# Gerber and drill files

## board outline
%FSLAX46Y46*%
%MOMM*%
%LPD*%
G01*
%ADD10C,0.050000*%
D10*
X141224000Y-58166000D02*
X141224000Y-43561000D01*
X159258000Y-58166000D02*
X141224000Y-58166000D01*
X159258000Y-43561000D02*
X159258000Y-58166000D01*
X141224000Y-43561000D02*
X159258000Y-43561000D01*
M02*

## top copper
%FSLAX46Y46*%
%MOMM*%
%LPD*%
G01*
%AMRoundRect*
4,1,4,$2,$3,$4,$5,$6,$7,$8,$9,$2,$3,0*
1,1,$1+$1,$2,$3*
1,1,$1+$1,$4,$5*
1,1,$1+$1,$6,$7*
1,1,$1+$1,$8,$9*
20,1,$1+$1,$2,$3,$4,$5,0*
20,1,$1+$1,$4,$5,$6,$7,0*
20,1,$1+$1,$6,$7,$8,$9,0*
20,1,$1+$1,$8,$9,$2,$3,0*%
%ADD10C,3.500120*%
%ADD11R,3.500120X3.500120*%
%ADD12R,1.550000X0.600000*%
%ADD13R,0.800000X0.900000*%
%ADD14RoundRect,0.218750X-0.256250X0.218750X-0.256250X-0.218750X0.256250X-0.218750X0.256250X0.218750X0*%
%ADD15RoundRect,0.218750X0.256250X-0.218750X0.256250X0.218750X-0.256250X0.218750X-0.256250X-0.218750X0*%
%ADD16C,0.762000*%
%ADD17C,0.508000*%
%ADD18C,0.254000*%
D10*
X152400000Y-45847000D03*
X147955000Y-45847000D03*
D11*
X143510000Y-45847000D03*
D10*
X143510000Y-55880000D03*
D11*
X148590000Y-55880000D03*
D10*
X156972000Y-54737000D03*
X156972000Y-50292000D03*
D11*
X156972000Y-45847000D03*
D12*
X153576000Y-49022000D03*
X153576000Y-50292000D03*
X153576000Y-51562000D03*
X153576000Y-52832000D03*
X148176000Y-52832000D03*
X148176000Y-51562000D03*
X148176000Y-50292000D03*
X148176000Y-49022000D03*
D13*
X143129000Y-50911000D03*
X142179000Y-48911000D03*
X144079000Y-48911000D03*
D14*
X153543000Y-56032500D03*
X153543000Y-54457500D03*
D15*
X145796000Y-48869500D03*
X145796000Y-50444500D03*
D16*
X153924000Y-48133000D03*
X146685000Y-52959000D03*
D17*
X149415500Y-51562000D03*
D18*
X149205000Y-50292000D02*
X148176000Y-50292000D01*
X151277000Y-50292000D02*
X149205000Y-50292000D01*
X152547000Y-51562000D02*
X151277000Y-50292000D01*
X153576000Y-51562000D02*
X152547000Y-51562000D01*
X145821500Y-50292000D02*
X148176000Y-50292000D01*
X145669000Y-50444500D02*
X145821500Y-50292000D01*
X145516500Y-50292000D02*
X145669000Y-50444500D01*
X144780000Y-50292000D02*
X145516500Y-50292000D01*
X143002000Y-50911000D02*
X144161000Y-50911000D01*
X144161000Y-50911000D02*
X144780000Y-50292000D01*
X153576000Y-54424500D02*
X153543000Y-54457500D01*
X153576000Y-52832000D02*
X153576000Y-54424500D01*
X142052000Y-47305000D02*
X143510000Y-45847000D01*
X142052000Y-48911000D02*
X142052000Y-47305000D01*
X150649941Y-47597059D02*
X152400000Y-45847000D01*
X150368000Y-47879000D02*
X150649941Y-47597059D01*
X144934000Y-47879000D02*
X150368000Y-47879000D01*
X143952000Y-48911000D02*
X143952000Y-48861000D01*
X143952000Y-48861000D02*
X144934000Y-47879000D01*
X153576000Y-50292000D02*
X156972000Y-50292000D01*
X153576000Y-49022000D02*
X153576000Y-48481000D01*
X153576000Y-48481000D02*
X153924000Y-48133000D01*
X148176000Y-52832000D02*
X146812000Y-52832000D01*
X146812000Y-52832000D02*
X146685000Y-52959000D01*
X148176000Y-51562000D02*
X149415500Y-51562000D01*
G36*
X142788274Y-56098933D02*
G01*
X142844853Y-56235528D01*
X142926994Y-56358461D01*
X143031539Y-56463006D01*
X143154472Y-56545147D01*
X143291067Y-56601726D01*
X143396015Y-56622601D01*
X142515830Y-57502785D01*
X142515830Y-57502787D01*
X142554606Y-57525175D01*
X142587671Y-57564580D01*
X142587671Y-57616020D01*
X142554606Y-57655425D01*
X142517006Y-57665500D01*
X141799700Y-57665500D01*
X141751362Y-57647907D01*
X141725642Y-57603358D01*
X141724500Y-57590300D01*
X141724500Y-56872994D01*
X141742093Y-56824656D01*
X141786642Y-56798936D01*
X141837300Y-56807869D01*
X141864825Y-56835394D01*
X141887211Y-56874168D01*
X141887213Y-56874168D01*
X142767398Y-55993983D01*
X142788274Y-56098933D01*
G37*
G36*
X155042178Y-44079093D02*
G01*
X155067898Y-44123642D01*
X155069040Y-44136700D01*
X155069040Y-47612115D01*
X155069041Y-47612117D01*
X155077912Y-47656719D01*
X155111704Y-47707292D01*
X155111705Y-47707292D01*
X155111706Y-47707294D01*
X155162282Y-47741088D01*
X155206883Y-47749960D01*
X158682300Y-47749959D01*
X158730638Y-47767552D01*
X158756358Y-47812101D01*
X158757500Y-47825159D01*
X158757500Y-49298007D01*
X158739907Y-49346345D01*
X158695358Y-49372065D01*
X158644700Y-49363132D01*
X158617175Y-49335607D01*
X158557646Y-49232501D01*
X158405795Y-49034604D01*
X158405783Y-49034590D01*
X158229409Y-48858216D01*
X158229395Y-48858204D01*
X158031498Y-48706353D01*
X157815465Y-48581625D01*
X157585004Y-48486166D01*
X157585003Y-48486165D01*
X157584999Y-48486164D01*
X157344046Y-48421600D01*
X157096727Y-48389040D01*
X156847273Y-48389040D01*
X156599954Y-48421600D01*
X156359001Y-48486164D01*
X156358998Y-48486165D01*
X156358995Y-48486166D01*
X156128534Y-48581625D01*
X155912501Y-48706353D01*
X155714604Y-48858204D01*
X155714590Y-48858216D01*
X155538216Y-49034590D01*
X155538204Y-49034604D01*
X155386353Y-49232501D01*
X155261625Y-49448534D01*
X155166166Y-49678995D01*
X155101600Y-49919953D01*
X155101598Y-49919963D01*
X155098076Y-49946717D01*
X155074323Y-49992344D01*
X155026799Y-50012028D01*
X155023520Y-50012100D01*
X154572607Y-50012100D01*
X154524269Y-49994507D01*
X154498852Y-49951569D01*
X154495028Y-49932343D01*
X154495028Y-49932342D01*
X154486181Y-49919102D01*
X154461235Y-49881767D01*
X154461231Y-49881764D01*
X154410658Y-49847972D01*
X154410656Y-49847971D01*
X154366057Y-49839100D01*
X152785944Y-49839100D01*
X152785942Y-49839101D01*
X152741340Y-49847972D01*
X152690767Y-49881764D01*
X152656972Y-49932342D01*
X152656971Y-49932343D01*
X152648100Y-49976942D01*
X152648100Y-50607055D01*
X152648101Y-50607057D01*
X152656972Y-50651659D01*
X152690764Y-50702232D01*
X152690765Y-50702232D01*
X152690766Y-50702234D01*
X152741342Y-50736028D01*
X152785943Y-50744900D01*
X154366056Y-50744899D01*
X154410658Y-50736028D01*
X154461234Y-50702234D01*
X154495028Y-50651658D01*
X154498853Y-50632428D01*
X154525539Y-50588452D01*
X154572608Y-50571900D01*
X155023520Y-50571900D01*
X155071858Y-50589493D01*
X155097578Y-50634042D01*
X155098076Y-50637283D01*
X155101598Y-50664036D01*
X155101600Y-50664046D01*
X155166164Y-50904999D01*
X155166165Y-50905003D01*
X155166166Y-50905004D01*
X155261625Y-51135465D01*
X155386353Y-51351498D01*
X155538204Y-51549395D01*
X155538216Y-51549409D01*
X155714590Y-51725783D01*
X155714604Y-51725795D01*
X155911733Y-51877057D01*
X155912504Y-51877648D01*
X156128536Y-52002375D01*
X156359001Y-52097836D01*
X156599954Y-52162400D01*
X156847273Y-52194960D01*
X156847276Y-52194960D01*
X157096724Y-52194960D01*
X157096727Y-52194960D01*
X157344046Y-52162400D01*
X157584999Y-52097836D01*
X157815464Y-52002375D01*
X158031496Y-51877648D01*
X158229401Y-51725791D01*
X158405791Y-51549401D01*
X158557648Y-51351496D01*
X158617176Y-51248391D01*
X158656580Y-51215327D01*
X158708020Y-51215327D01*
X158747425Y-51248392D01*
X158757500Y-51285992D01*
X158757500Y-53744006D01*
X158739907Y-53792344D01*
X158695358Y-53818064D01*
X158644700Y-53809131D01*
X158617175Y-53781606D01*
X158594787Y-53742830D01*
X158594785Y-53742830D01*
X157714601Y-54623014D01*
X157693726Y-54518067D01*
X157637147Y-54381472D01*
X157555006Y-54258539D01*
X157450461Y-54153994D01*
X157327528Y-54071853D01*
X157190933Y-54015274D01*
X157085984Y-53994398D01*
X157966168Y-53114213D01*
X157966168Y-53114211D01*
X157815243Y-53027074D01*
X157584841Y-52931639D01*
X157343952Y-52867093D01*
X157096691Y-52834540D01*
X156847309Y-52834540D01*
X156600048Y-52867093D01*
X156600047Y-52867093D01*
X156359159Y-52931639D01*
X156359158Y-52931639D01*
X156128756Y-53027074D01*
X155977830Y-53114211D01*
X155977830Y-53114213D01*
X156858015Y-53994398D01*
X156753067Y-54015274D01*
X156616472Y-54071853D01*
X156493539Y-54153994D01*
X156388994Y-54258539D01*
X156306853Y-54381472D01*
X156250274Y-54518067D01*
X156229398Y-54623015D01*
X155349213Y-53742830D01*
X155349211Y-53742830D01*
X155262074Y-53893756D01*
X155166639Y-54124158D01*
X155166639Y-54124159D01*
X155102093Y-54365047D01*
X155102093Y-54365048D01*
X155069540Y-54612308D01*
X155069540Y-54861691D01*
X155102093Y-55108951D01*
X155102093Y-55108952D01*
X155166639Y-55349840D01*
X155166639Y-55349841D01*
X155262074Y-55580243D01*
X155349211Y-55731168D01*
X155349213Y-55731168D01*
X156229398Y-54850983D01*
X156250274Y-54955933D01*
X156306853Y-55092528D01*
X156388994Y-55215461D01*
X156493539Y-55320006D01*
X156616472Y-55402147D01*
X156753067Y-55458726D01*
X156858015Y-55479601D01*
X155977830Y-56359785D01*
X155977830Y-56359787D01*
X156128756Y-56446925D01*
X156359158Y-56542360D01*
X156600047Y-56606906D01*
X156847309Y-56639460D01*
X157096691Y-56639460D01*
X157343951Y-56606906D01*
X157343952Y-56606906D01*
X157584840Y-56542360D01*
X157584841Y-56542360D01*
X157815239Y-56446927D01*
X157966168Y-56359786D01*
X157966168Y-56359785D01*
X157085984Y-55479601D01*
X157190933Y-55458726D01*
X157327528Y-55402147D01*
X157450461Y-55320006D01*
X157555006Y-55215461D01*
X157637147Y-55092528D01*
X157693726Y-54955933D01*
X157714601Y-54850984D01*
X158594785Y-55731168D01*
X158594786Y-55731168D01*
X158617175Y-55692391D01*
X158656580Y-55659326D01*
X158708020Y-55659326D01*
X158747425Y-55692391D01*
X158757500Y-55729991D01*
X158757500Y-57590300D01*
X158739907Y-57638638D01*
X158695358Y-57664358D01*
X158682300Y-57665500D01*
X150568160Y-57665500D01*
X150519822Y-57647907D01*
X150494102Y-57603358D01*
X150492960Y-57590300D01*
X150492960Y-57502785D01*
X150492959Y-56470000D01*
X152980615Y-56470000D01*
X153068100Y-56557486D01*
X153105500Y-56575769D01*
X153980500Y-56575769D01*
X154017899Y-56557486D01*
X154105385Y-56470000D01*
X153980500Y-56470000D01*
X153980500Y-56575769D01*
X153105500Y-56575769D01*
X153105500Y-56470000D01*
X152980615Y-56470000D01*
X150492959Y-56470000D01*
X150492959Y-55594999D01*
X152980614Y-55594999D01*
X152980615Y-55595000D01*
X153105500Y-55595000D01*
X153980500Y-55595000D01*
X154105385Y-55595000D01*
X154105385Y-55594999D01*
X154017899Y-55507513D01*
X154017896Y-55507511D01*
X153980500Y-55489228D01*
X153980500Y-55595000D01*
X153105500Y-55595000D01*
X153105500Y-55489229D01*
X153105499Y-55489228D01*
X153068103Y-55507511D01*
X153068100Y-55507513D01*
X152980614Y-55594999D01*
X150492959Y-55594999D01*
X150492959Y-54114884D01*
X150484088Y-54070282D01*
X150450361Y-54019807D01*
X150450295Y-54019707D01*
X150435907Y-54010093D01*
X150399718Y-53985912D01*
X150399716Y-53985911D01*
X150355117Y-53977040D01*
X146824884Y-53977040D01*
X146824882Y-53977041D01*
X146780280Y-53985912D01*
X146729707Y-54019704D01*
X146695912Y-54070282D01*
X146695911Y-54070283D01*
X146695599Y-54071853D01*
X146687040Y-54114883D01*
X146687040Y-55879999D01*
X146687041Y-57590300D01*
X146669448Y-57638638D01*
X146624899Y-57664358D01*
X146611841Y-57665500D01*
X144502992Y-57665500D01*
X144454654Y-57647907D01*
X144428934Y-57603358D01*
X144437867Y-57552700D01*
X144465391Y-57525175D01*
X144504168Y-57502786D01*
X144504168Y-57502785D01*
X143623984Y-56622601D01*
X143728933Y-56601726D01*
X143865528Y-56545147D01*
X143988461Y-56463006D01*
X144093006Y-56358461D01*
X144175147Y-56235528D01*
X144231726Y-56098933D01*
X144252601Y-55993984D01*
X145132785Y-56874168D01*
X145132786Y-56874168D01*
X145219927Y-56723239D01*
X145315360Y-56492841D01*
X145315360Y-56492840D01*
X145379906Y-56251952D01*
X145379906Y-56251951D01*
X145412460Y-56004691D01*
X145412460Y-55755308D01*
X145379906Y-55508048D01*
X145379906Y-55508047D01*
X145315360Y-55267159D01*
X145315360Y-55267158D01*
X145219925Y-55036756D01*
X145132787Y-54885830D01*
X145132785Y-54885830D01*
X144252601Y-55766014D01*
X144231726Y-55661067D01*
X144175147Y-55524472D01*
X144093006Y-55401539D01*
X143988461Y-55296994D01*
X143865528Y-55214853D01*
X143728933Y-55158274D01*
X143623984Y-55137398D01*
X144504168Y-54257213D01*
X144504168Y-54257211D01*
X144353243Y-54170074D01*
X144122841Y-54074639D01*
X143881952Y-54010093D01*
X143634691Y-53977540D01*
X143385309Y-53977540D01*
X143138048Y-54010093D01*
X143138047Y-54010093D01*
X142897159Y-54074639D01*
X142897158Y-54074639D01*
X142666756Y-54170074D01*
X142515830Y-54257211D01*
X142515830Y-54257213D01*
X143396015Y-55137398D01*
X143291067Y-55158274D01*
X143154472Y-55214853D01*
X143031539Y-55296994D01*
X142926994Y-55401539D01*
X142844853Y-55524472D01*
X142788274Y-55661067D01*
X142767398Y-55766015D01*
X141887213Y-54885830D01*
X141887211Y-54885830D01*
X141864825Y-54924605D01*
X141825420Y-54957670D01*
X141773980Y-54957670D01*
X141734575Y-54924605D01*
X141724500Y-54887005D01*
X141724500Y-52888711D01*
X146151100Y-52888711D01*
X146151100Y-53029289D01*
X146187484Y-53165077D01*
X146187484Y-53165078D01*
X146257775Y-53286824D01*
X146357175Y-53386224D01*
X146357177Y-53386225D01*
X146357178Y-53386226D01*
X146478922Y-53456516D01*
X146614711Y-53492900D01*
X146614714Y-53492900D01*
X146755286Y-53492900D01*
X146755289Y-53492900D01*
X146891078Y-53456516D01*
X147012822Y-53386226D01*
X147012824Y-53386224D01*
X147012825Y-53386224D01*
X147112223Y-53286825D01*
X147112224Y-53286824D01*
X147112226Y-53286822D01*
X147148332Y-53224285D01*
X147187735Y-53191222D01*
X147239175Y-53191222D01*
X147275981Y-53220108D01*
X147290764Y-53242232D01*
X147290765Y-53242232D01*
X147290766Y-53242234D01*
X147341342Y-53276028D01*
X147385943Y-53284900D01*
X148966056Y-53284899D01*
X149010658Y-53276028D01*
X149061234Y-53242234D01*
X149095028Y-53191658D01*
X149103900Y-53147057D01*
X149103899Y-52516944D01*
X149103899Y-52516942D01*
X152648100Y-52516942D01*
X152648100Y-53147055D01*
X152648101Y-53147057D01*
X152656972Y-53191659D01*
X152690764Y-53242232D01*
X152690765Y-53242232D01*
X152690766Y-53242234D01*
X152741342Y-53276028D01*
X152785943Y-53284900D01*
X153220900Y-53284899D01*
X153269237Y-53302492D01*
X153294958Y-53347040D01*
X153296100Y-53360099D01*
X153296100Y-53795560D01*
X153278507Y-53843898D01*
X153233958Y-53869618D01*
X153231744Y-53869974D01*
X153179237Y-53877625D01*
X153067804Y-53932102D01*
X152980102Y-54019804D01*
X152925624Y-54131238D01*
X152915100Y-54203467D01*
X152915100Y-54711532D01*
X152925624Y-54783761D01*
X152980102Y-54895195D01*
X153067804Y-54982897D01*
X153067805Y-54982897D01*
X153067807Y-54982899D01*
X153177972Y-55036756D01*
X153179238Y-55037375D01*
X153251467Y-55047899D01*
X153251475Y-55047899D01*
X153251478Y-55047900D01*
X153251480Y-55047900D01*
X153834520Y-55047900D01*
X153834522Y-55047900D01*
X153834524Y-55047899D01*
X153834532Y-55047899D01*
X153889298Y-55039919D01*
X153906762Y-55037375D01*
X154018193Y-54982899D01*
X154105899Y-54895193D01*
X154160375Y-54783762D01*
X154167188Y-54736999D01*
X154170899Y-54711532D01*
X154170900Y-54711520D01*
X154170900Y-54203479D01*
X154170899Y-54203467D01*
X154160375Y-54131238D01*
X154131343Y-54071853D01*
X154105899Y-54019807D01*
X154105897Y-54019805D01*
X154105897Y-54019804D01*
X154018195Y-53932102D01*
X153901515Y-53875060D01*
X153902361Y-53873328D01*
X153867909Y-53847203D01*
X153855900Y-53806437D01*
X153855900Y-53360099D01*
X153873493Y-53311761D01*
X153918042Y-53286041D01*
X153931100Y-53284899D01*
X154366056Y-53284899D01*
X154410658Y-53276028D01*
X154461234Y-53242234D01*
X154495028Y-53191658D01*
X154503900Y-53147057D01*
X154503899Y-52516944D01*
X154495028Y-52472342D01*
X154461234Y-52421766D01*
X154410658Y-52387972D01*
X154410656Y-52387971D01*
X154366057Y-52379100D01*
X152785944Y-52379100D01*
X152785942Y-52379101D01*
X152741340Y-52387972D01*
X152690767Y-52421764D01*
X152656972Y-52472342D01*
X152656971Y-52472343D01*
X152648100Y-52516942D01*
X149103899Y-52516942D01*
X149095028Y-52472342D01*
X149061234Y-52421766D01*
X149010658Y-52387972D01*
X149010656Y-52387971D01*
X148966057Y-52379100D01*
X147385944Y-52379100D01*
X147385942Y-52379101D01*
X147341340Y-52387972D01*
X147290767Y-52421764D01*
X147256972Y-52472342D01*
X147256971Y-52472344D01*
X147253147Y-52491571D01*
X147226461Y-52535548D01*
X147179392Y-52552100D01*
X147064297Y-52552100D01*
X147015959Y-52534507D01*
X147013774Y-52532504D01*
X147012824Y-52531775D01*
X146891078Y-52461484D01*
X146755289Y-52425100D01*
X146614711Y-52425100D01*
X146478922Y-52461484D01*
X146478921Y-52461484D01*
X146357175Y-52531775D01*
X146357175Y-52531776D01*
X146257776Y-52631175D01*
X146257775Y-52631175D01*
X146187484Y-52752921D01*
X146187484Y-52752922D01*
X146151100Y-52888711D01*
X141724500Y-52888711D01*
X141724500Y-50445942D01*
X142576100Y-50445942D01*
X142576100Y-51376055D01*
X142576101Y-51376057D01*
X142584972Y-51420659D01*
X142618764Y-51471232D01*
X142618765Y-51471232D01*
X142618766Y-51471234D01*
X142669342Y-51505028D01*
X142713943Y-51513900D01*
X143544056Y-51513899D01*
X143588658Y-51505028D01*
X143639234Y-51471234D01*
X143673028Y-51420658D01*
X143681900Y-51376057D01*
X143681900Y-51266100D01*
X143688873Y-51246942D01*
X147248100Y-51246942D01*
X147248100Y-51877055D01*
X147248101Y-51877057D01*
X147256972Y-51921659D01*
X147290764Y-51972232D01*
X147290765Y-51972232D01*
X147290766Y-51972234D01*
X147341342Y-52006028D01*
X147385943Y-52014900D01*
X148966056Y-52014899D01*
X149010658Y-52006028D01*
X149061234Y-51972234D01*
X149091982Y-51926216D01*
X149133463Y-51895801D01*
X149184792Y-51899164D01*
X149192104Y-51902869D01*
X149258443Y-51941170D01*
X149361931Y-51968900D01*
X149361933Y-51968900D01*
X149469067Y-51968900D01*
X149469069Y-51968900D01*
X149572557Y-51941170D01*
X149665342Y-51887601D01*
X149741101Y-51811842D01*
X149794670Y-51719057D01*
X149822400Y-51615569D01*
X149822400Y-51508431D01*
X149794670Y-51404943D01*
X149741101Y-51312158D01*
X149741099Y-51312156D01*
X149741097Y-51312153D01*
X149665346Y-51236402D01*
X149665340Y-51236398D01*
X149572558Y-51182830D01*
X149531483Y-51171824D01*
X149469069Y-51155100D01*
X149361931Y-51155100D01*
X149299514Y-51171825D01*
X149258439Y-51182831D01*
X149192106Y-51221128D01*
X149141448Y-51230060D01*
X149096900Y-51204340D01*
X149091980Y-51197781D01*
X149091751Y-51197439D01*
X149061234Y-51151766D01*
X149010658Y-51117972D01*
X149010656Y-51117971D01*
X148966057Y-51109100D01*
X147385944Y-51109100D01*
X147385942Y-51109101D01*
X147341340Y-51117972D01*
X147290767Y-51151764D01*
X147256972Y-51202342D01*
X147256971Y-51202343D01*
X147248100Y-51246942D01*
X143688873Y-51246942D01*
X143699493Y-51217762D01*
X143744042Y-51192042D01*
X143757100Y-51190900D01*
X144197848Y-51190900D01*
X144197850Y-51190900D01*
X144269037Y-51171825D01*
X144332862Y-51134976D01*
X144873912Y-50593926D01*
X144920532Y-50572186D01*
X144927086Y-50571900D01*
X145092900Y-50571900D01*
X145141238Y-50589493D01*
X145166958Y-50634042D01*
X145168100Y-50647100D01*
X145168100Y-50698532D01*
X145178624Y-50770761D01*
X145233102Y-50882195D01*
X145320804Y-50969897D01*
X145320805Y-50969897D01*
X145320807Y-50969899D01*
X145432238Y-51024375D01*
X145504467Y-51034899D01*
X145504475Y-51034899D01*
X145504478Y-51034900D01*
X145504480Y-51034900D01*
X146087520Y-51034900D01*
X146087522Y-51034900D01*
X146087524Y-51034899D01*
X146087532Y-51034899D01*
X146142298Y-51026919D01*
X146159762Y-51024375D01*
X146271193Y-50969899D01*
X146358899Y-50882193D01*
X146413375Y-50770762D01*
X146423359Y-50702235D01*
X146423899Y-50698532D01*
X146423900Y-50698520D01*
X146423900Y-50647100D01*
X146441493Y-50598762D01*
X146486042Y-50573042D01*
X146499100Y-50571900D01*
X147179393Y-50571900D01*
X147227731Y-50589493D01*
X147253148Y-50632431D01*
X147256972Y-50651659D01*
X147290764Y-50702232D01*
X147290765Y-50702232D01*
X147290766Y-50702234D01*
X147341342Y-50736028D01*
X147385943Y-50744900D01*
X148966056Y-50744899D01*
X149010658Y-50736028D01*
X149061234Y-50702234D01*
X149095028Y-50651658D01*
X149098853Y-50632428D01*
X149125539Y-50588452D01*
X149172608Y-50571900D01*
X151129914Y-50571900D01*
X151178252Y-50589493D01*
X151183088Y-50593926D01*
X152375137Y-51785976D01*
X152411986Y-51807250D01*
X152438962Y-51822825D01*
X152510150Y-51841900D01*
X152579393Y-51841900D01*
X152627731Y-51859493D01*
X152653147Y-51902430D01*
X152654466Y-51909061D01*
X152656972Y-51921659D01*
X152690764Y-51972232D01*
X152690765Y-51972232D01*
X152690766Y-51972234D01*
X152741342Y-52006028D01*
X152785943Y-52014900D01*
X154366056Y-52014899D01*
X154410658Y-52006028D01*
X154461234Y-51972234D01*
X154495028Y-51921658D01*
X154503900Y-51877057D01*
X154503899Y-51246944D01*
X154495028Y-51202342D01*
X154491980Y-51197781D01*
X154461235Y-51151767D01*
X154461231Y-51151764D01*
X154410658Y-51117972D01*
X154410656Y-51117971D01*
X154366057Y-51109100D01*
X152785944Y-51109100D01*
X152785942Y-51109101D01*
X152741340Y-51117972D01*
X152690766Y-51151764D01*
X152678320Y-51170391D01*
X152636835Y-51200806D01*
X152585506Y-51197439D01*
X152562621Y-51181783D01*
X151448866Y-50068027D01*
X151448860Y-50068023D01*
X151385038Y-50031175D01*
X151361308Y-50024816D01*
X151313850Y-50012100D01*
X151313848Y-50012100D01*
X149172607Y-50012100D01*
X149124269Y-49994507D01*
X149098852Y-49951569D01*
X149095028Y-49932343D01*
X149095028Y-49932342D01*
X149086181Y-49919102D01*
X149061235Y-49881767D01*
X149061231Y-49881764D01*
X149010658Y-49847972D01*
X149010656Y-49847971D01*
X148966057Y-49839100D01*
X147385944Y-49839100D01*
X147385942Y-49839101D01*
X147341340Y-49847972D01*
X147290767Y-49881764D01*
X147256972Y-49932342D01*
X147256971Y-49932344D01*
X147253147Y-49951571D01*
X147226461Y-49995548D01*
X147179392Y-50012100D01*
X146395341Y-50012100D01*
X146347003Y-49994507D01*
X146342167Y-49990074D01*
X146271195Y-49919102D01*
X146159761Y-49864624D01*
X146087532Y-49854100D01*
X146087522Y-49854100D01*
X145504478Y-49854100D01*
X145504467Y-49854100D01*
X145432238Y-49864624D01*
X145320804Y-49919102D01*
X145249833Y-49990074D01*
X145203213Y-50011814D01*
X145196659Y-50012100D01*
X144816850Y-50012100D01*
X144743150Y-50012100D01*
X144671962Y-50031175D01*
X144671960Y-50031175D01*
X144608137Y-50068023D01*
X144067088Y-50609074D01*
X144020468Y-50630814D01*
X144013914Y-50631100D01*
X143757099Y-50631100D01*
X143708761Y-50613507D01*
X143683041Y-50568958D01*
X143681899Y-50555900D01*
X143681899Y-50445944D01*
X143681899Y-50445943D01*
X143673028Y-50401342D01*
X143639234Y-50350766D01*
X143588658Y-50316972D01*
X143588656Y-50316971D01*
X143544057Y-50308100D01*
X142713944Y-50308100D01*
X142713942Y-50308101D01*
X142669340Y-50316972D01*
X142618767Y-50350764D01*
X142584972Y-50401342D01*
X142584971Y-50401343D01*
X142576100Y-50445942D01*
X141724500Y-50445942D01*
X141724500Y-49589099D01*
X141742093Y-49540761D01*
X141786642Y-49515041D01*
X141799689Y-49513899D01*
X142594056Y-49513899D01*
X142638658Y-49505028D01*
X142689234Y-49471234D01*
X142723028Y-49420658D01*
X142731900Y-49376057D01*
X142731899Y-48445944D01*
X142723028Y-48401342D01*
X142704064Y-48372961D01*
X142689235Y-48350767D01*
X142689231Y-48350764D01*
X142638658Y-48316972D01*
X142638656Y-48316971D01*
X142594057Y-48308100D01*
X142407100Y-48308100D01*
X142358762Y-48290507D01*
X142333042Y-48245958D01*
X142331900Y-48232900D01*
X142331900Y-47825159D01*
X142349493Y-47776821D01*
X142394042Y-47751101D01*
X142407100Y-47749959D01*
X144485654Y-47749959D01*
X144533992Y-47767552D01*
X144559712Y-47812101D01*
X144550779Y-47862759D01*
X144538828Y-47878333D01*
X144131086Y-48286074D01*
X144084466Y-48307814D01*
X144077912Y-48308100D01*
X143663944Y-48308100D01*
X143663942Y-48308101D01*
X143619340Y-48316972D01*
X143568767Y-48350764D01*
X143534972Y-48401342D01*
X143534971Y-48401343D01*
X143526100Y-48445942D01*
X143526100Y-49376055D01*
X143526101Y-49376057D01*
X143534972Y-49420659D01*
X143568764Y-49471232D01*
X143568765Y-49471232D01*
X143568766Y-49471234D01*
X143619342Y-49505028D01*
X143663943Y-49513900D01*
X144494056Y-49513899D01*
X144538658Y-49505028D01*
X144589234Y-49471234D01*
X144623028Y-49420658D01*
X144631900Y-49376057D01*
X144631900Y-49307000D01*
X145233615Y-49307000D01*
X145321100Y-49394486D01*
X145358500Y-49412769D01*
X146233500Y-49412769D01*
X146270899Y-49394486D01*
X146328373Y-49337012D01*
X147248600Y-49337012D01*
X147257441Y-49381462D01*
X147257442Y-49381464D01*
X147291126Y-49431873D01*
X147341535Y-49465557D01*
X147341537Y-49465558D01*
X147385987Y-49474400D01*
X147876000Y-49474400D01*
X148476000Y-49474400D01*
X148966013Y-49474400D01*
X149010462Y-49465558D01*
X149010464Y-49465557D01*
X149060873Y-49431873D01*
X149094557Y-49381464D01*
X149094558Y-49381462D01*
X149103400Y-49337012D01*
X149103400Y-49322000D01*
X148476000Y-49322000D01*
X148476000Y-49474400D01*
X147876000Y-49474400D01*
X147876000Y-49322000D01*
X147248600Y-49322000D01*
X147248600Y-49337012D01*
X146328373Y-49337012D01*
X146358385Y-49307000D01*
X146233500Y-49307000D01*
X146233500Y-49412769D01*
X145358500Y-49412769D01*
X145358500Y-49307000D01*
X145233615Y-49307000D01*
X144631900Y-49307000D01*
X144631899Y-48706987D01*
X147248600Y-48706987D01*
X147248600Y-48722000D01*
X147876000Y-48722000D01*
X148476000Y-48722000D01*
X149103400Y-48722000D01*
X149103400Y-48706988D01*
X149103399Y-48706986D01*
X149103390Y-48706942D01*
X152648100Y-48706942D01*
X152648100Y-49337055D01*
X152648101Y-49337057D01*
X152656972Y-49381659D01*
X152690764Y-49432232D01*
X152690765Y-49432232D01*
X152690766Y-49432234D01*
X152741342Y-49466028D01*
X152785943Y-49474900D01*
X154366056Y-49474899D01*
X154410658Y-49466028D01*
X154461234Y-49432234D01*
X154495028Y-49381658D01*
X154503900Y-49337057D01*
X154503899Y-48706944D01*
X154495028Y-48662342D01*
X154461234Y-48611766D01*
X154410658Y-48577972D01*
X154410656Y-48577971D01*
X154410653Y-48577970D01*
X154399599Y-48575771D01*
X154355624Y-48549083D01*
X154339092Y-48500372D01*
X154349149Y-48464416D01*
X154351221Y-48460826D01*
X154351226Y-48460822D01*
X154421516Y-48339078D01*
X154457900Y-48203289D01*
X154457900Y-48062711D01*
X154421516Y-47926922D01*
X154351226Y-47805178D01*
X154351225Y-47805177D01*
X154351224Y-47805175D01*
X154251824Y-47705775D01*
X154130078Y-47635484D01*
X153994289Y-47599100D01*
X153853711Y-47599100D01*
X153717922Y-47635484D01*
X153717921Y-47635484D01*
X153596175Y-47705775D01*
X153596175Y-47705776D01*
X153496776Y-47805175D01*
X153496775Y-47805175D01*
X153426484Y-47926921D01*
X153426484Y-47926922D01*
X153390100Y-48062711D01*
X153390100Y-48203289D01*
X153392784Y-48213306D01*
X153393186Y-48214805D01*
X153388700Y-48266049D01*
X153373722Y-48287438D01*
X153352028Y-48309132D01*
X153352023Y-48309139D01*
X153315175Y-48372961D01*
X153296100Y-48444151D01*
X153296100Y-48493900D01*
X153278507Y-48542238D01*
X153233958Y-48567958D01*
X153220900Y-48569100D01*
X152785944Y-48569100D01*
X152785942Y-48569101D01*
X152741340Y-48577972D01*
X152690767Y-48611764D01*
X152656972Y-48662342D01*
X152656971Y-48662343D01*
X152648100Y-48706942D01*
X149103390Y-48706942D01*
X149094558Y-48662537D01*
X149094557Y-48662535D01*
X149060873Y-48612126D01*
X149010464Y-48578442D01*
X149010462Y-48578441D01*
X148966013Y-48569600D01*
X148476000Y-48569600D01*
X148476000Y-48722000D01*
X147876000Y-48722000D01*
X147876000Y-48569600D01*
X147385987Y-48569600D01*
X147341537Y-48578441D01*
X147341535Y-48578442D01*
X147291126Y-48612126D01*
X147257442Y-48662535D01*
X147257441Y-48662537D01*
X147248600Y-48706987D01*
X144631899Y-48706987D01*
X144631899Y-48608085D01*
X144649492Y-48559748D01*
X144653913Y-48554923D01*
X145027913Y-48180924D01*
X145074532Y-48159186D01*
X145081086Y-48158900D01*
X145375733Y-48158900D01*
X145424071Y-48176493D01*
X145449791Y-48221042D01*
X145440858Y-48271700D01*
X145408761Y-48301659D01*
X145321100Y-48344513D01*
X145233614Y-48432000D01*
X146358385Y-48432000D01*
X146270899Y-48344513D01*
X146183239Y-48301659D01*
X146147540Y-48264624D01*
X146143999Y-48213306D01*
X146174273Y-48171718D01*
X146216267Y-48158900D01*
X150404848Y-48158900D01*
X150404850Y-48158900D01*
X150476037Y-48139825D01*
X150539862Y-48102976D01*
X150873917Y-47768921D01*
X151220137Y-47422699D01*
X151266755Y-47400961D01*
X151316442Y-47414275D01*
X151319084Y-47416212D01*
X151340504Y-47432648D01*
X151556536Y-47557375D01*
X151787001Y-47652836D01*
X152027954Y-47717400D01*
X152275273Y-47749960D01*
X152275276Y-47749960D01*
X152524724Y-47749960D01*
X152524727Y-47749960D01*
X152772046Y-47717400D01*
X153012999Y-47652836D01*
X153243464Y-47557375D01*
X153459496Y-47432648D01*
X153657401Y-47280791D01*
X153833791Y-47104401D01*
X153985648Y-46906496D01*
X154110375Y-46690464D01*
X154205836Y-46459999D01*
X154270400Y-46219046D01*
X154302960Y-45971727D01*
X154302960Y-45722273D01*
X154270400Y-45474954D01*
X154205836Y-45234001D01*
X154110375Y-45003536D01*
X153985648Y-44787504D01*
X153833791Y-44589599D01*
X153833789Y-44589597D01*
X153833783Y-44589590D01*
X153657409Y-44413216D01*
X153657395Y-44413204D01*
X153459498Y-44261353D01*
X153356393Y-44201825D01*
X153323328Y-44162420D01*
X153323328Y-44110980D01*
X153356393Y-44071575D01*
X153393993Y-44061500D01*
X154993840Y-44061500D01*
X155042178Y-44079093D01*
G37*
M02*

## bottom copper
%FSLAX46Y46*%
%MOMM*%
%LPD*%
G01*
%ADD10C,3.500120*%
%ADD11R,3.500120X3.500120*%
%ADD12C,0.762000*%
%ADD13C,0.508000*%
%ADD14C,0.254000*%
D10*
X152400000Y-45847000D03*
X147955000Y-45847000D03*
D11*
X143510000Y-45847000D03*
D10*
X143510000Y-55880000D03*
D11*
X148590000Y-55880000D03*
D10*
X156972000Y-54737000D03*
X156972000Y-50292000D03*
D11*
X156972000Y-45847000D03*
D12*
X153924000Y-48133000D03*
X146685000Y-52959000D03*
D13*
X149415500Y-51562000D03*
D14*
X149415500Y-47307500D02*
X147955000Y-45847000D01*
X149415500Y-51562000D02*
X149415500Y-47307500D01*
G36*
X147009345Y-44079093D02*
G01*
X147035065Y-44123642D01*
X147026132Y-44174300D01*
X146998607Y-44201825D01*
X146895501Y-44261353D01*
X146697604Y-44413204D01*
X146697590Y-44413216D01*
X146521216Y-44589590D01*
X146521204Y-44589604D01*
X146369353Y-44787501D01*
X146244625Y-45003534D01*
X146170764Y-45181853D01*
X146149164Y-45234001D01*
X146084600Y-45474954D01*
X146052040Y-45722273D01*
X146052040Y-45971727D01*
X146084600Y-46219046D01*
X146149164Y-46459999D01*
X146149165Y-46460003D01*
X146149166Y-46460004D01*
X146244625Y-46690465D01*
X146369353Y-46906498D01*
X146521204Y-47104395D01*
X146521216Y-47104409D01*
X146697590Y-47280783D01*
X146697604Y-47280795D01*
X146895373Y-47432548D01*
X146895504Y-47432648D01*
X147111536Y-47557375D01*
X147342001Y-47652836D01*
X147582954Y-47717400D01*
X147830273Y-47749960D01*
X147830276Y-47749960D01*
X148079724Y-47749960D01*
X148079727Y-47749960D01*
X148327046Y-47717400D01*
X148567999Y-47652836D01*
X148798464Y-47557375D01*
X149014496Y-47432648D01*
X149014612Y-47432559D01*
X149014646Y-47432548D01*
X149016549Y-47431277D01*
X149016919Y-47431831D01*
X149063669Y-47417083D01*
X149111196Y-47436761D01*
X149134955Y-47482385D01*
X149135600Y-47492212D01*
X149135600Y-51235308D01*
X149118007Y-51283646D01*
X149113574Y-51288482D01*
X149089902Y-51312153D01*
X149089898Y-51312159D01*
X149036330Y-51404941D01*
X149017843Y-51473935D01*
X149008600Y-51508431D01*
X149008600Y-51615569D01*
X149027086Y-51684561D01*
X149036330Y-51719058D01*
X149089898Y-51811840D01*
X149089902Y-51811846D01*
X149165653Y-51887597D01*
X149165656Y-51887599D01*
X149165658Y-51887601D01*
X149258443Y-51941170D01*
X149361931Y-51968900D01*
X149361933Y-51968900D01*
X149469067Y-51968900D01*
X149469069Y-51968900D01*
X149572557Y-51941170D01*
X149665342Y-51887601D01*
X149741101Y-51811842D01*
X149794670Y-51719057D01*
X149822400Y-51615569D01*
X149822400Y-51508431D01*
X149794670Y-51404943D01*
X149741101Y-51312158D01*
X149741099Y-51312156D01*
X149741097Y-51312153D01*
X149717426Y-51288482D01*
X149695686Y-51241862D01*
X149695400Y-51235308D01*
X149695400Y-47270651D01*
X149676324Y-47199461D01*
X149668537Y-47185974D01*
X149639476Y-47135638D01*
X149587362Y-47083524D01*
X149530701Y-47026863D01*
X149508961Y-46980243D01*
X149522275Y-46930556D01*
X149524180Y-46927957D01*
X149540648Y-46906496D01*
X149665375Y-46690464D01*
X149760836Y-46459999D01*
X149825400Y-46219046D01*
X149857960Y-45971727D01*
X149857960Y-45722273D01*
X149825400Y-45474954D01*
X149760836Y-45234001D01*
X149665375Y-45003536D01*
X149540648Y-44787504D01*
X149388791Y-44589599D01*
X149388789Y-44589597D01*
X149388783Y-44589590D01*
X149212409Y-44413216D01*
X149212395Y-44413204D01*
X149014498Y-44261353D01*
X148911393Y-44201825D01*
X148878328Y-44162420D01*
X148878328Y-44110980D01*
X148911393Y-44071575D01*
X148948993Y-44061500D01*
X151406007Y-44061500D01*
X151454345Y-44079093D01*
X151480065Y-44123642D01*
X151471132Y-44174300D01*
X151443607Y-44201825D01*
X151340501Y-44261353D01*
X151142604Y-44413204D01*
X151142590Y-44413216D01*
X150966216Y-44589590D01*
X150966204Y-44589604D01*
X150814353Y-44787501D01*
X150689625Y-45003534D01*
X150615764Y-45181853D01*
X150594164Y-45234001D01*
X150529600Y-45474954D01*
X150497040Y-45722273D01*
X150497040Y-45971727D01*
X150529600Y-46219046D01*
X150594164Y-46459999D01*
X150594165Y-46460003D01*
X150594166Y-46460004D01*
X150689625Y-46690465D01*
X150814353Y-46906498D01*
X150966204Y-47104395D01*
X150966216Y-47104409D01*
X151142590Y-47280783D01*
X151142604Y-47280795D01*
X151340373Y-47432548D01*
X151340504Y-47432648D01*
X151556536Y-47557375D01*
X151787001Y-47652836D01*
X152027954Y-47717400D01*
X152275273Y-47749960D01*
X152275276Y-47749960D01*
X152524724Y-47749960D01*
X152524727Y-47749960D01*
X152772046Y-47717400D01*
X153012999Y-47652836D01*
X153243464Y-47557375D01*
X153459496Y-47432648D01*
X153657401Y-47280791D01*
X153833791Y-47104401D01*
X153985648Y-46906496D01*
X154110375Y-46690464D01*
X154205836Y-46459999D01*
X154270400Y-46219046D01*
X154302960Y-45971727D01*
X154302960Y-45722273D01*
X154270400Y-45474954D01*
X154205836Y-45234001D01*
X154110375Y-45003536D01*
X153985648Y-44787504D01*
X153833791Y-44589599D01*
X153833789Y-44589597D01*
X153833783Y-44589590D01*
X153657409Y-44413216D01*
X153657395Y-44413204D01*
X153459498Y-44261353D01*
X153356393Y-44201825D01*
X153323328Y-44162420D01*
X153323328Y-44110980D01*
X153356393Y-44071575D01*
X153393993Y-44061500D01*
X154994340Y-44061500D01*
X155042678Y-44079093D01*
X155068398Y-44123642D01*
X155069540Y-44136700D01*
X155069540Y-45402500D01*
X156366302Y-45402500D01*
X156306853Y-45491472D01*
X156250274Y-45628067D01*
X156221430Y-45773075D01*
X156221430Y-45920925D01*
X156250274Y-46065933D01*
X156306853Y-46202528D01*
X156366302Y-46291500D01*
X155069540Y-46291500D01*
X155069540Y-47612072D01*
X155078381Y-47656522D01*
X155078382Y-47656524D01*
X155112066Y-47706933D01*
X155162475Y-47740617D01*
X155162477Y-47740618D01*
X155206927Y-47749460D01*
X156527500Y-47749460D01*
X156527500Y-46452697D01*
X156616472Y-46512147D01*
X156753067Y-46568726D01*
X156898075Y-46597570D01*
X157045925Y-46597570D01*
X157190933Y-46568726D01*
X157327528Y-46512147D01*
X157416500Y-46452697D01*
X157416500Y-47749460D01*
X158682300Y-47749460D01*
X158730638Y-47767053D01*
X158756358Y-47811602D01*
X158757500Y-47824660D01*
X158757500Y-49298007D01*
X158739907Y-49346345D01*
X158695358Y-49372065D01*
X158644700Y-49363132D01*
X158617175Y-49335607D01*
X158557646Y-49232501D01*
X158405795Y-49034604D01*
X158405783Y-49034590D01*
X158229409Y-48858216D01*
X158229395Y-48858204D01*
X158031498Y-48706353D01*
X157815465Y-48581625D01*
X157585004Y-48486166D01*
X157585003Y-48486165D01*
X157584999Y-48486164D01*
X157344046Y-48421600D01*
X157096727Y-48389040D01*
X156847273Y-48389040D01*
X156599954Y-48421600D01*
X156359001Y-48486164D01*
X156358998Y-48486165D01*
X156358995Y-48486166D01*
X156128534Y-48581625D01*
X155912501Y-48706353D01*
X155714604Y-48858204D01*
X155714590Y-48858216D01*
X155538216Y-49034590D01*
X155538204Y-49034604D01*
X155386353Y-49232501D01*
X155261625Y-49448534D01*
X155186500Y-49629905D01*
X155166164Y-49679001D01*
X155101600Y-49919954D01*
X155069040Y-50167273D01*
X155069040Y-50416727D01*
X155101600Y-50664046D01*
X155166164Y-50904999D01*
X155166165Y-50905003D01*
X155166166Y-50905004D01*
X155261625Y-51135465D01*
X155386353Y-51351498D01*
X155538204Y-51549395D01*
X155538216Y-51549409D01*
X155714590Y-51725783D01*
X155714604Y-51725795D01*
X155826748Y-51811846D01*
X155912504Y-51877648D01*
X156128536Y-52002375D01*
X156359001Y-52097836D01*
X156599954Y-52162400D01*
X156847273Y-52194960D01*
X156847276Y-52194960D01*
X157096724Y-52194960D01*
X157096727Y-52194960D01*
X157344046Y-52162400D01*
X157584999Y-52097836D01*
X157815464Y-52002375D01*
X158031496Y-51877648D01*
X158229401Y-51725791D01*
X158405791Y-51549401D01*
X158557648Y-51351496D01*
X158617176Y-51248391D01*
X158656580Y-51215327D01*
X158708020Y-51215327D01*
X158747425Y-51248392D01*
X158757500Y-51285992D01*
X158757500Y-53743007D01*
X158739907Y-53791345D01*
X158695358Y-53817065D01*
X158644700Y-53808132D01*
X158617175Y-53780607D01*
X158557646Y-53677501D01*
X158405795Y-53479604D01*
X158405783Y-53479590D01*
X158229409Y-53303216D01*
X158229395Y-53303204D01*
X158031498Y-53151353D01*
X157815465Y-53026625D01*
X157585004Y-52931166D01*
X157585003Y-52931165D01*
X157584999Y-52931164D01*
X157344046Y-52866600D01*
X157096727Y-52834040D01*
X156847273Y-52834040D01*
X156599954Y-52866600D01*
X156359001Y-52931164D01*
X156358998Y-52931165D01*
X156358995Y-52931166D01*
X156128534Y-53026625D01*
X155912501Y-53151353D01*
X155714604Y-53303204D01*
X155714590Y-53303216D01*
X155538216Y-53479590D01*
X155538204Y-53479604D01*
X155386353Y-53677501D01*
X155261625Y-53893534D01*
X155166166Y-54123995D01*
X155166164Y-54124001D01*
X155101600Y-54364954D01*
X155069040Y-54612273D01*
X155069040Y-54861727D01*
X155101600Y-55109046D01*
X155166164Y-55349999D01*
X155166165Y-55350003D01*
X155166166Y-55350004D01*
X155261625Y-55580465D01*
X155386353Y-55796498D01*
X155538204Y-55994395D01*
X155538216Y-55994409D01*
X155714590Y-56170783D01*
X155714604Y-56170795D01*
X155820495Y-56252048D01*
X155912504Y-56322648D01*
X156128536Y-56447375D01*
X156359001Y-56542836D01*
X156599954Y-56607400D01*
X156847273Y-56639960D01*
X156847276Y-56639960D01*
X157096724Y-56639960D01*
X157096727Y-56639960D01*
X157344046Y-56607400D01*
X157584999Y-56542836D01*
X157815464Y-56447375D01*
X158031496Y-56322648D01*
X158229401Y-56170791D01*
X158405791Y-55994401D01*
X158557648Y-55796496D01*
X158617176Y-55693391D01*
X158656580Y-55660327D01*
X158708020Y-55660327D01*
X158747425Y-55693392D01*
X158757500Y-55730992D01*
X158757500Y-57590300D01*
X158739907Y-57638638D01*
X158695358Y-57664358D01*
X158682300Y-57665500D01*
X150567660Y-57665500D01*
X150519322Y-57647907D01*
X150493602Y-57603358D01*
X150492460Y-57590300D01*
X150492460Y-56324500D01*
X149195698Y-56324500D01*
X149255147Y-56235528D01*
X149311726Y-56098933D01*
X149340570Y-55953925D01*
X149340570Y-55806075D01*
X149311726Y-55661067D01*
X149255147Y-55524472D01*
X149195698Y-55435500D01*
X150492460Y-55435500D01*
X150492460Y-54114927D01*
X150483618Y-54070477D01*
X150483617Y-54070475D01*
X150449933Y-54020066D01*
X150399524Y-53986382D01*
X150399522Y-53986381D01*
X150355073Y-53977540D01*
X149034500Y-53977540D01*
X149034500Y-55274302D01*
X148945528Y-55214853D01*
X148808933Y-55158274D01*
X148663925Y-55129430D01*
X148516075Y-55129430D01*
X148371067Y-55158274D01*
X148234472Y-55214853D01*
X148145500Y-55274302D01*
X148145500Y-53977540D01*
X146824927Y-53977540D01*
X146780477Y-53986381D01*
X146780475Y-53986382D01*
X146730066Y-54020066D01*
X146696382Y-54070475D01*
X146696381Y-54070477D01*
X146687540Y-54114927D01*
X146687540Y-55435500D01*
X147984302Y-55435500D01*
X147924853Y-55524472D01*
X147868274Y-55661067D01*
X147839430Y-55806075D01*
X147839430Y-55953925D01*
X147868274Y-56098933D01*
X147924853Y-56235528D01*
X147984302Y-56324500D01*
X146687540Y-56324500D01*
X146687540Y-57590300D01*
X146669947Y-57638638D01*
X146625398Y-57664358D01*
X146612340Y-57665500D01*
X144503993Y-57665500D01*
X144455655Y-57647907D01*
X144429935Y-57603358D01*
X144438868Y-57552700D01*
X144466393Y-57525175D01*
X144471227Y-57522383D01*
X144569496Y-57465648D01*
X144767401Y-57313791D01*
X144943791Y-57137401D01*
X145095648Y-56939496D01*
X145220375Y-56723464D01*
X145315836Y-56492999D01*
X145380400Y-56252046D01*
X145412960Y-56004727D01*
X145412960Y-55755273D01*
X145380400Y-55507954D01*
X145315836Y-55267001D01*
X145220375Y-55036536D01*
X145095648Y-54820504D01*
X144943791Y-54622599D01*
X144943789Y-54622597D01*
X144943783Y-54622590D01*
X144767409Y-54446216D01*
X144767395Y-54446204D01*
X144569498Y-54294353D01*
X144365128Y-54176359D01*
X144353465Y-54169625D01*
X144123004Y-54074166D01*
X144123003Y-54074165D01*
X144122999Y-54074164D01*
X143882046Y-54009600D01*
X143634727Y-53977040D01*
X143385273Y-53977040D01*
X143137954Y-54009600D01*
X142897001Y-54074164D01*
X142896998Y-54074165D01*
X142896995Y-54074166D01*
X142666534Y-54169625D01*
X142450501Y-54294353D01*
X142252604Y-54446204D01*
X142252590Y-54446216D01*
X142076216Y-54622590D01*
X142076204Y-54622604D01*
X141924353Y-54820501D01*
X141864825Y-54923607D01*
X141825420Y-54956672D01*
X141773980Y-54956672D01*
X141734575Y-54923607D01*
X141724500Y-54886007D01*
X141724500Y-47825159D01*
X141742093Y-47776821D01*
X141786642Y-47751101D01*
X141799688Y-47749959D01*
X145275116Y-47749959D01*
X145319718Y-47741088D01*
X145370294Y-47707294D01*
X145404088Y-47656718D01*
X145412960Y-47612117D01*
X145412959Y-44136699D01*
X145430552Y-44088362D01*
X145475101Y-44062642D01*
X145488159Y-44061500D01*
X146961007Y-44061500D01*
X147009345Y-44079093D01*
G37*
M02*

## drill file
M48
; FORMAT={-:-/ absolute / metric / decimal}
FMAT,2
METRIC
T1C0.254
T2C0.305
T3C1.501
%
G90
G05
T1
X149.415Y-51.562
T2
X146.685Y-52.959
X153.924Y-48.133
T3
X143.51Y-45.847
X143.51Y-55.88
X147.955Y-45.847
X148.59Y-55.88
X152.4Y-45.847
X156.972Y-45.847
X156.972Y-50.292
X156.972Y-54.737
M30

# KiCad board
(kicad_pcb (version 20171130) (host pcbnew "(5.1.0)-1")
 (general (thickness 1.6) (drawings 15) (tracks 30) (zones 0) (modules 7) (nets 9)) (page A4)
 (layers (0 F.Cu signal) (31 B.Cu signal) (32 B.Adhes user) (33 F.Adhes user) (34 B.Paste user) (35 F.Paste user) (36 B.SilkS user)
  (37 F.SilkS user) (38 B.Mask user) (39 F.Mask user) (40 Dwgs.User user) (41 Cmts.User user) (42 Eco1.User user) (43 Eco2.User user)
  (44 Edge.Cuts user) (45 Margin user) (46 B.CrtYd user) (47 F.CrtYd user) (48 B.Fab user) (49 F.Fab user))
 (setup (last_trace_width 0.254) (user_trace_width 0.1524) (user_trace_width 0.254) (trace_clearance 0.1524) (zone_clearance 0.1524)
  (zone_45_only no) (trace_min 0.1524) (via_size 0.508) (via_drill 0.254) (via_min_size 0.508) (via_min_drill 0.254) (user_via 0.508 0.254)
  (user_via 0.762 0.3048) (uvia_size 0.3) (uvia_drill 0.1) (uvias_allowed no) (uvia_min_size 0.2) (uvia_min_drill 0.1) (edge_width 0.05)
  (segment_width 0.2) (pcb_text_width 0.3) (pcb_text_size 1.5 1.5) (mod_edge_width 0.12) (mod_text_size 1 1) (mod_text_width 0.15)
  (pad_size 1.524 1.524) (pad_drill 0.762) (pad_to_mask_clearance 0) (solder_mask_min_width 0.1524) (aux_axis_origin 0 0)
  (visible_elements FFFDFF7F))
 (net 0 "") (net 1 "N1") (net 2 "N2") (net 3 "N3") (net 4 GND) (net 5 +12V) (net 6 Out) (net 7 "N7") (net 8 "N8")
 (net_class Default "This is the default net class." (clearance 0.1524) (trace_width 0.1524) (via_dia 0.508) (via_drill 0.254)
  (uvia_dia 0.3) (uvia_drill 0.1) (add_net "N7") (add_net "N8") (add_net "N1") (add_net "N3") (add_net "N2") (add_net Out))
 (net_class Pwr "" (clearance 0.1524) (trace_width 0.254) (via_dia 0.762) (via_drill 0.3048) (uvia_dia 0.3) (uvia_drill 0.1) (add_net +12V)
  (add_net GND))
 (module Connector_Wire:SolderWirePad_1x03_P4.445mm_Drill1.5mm (layer F.Cu) (at 143.51 45.847)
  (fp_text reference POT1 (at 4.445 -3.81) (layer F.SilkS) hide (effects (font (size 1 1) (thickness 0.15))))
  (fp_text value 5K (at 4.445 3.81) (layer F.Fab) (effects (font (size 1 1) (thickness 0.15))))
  (pad 3 thru_hole circle (at 8.89 0) (size 3.50012 3.50012) (drill 1.50114) (layers *.Cu *.Mask) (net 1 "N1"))
  (pad 2 thru_hole circle (at 4.445 0) (size 3.50012 3.50012) (drill 1.50114) (layers *.Cu *.Mask) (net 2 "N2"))
  (pad 1 thru_hole rect (at 0 0) (size 3.50012 3.50012) (drill 1.50114) (layers *.Cu *.Mask) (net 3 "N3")))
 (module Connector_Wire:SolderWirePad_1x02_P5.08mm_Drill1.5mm (layer F.Cu) (at 148.59 55.88 180)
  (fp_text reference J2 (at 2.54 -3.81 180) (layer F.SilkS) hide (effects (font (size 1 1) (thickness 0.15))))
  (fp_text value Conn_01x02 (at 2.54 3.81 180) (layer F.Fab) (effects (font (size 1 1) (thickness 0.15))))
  (pad 2 thru_hole circle (at 5.08 0 180) (size 3.50012 3.50012) (drill 1.50114) (layers *.Cu *.Mask) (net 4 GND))
  (pad 1 thru_hole rect (at 0 0 180) (size 3.50012 3.50012) (drill 1.50114) (layers *.Cu *.Mask) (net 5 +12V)))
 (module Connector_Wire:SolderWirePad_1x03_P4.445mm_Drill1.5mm (layer F.Cu) (at 156.972 45.847 270)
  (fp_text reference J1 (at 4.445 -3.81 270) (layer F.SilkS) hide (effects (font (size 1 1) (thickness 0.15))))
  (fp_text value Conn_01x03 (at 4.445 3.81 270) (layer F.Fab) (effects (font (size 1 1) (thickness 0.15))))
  (pad 3 thru_hole circle (at 8.89 0 270) (size 3.50012 3.50012) (drill 1.50114) (layers *.Cu *.Mask) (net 4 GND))
  (pad 2 thru_hole circle (at 4.445 0 270) (size 3.50012 3.50012) (drill 1.50114) (layers *.Cu *.Mask) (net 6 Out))
  (pad 1 thru_hole rect (at 0 0 270) (size 3.50012 3.50012) (drill 1.50114) (layers *.Cu *.Mask) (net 5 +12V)))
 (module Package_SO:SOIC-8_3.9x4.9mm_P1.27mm (layer F.Cu) (at 150.876 50.927)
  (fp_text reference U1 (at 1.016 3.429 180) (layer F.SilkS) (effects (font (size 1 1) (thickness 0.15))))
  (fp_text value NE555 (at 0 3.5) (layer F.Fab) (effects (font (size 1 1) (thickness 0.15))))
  (pad 8 smd rect (at 2.7 -1.905) (size 1.55 0.6) (layers F.Cu F.Paste F.Mask) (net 5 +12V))
  (pad 7 smd rect (at 2.7 -0.635) (size 1.55 0.6) (layers F.Cu F.Paste F.Mask) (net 6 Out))
  (pad 6 smd rect (at 2.7 0.635) (size 1.55 0.6) (layers F.Cu F.Paste F.Mask) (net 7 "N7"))
  (pad 5 smd rect (at 2.7 1.905) (size 1.55 0.6) (layers F.Cu F.Paste F.Mask) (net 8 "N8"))
  (pad 4 smd rect (at -2.7 1.905) (size 1.55 0.6) (layers F.Cu F.Paste F.Mask) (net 5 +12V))
  (pad 3 smd rect (at -2.7 0.635) (size 1.55 0.6) (layers F.Cu F.Paste F.Mask) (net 2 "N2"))
  (pad 2 smd rect (at -2.7 -0.635) (size 1.55 0.6) (layers F.Cu F.Paste F.Mask) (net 7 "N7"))
  (pad 1 smd rect (at -2.7 -1.905) (size 1.55 0.6) (layers F.Cu F.Paste F.Mask) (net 4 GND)))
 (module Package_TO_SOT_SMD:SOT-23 (layer F.Cu) (at 143.129 49.911 270)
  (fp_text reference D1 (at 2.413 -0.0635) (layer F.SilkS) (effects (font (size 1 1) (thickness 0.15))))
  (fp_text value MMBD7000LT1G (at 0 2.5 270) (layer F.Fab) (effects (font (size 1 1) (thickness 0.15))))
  (pad 3 smd rect (at 1 0 270) (size 0.9 0.8) (layers F.Cu F.Paste F.Mask) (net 7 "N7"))
  (pad 2 smd rect (at -1 0.95 270) (size 0.9 0.8) (layers F.Cu F.Paste F.Mask) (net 3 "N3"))
  (pad 1 smd rect (at -1 -0.95 270) (size 0.9 0.8) (layers F.Cu F.Paste F.Mask) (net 1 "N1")))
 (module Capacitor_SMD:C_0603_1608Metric (layer F.Cu) (at 153.543 55.245 270)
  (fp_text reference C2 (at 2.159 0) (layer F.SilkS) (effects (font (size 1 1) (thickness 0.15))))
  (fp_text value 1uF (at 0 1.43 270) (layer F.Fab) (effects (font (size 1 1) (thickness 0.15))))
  (pad 2 smd roundrect (at 0.7875 0 270) (size 0.875 0.95) (layers F.Cu F.Paste F.Mask) (roundrect_rratio 0.25) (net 4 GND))
  (pad 1 smd roundrect (at -0.7875 0 270) (size 0.875 0.95) (layers F.Cu F.Paste F.Mask) (roundrect_rratio 0.25) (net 8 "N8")))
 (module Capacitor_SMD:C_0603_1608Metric (layer F.Cu) (at 145.796 49.657 90)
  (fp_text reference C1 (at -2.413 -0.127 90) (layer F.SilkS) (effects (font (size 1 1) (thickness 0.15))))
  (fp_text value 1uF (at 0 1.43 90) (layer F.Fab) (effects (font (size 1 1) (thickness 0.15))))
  (pad 2 smd roundrect (at 0.7875 0 90) (size 0.875 0.95) (layers F.Cu F.Paste F.Mask) (roundrect_rratio 0.25) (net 4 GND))
  (pad 1 smd roundrect (at -0.7875 0 90) (size 0.875 0.95) (layers F.Cu F.Paste F.Mask) (roundrect_rratio 0.25) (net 7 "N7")))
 (gr_line (start 141.224 58.166) (end 141.224 43.561) (layer Edge.Cuts) (width 0.05))
 (gr_line (start 159.258 58.166) (end 141.224 58.166) (layer Edge.Cuts) (width 0.05))
 (gr_line (start 159.258 43.561) (end 159.258 58.166) (layer Edge.Cuts) (width 0.05))
 (gr_line (start 141.224 43.561) (end 159.258 43.561) (layer Edge.Cuts) (width 0.05))
 (segment (start 149.205 50.292) (end 148.176 50.292) (width 0.254) (layer F.Cu) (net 7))
 (segment (start 151.277 50.292) (end 149.205 50.292) (width 0.254) (layer F.Cu) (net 7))
 (segment (start 152.547 51.562) (end 151.277 50.292) (width 0.254) (layer F.Cu) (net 7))
 (segment (start 153.576 51.562) (end 152.547 51.562) (width 0.254) (layer F.Cu) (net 7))
 (segment (start 145.8215 50.292) (end 148.176 50.292) (width 0.254) (layer F.Cu) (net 7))
 (segment (start 145.669 50.4445) (end 145.8215 50.292) (width 0.254) (layer F.Cu) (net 7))
 (segment (start 145.5165 50.292) (end 145.669 50.4445) (width 0.254) (layer F.Cu) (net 7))
 (segment (start 144.78 50.292) (end 145.5165 50.292) (width 0.254) (layer F.Cu) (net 7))
 (segment (start 143.002 50.911) (end 144.161 50.911) (width 0.254) (layer F.Cu) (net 7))
 (segment (start 144.161 50.911) (end 144.78 50.292) (width 0.254) (layer F.Cu) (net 7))
 (segment (start 153.576 54.4245) (end 153.543 54.4575) (width 0.254) (layer F.Cu) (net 8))
 (segment (start 153.576 52.832) (end 153.576 54.4245) (width 0.254) (layer F.Cu) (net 8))
 (segment (start 142.052 47.305) (end 143.51 45.847) (width 0.254) (layer F.Cu) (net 3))
 (segment (start 142.052 48.911) (end 142.052 47.305) (width 0.254) (layer F.Cu) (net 3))
 (segment (start 150.649941 47.597059) (end 152.4 45.847) (width 0.254) (layer F.Cu) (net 1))
 (segment (start 150.368 47.879) (end 150.649941 47.597059) (width 0.254) (layer F.Cu) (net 1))
 (segment (start 144.934 47.879) (end 150.368 47.879) (width 0.254) (layer F.Cu) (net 1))
 (segment (start 143.952 48.911) (end 143.952 48.861) (width 0.254) (layer F.Cu) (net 1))
 (segment (start 143.952 48.861) (end 144.934 47.879) (width 0.254) (layer F.Cu) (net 1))
 (segment (start 153.576 50.292) (end 156.972 50.292) (width 0.254) (layer F.Cu) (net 6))
 (via (at 153.924 48.133) (size 0.762) (drill 0.3048) (layers F.Cu B.Cu) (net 5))
 (segment (start 153.576 49.022) (end 153.576 48.481) (width 0.254) (layer F.Cu) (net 5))
 (segment (start 153.576 48.481) (end 153.924 48.133) (width 0.254) (layer F.Cu) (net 5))
 (via (at 146.685 52.959) (size 0.762) (drill 0.3048) (layers F.Cu B.Cu) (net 5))
 (segment (start 148.176 52.832) (end 146.812 52.832) (width 0.254) (layer F.Cu) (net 5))
 (segment (start 146.812 52.832) (end 146.685 52.959) (width 0.254) (layer F.Cu) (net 5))
 (via (at 149.4155 51.562) (size 0.508) (drill 0.254) (layers F.Cu B.Cu) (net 2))
 (segment (start 148.176 51.562) (end 149.4155 51.562) (width 0.254) (layer F.Cu) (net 2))
 (segment (start 149.4155 47.3075) (end 147.955 45.847) (width 0.254) (layer B.Cu) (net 2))
 (segment (start 149.4155 51.562) (end 149.4155 47.3075) (width 0.254) (layer B.Cu) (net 2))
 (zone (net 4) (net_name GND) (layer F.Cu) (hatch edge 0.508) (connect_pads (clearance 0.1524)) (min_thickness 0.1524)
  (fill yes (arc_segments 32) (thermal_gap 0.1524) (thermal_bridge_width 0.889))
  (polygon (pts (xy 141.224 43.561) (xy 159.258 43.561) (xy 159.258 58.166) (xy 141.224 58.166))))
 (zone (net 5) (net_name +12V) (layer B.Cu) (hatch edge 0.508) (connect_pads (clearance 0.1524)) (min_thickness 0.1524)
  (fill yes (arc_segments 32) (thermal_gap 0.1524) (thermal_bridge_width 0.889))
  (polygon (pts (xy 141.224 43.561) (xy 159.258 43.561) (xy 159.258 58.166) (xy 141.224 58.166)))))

